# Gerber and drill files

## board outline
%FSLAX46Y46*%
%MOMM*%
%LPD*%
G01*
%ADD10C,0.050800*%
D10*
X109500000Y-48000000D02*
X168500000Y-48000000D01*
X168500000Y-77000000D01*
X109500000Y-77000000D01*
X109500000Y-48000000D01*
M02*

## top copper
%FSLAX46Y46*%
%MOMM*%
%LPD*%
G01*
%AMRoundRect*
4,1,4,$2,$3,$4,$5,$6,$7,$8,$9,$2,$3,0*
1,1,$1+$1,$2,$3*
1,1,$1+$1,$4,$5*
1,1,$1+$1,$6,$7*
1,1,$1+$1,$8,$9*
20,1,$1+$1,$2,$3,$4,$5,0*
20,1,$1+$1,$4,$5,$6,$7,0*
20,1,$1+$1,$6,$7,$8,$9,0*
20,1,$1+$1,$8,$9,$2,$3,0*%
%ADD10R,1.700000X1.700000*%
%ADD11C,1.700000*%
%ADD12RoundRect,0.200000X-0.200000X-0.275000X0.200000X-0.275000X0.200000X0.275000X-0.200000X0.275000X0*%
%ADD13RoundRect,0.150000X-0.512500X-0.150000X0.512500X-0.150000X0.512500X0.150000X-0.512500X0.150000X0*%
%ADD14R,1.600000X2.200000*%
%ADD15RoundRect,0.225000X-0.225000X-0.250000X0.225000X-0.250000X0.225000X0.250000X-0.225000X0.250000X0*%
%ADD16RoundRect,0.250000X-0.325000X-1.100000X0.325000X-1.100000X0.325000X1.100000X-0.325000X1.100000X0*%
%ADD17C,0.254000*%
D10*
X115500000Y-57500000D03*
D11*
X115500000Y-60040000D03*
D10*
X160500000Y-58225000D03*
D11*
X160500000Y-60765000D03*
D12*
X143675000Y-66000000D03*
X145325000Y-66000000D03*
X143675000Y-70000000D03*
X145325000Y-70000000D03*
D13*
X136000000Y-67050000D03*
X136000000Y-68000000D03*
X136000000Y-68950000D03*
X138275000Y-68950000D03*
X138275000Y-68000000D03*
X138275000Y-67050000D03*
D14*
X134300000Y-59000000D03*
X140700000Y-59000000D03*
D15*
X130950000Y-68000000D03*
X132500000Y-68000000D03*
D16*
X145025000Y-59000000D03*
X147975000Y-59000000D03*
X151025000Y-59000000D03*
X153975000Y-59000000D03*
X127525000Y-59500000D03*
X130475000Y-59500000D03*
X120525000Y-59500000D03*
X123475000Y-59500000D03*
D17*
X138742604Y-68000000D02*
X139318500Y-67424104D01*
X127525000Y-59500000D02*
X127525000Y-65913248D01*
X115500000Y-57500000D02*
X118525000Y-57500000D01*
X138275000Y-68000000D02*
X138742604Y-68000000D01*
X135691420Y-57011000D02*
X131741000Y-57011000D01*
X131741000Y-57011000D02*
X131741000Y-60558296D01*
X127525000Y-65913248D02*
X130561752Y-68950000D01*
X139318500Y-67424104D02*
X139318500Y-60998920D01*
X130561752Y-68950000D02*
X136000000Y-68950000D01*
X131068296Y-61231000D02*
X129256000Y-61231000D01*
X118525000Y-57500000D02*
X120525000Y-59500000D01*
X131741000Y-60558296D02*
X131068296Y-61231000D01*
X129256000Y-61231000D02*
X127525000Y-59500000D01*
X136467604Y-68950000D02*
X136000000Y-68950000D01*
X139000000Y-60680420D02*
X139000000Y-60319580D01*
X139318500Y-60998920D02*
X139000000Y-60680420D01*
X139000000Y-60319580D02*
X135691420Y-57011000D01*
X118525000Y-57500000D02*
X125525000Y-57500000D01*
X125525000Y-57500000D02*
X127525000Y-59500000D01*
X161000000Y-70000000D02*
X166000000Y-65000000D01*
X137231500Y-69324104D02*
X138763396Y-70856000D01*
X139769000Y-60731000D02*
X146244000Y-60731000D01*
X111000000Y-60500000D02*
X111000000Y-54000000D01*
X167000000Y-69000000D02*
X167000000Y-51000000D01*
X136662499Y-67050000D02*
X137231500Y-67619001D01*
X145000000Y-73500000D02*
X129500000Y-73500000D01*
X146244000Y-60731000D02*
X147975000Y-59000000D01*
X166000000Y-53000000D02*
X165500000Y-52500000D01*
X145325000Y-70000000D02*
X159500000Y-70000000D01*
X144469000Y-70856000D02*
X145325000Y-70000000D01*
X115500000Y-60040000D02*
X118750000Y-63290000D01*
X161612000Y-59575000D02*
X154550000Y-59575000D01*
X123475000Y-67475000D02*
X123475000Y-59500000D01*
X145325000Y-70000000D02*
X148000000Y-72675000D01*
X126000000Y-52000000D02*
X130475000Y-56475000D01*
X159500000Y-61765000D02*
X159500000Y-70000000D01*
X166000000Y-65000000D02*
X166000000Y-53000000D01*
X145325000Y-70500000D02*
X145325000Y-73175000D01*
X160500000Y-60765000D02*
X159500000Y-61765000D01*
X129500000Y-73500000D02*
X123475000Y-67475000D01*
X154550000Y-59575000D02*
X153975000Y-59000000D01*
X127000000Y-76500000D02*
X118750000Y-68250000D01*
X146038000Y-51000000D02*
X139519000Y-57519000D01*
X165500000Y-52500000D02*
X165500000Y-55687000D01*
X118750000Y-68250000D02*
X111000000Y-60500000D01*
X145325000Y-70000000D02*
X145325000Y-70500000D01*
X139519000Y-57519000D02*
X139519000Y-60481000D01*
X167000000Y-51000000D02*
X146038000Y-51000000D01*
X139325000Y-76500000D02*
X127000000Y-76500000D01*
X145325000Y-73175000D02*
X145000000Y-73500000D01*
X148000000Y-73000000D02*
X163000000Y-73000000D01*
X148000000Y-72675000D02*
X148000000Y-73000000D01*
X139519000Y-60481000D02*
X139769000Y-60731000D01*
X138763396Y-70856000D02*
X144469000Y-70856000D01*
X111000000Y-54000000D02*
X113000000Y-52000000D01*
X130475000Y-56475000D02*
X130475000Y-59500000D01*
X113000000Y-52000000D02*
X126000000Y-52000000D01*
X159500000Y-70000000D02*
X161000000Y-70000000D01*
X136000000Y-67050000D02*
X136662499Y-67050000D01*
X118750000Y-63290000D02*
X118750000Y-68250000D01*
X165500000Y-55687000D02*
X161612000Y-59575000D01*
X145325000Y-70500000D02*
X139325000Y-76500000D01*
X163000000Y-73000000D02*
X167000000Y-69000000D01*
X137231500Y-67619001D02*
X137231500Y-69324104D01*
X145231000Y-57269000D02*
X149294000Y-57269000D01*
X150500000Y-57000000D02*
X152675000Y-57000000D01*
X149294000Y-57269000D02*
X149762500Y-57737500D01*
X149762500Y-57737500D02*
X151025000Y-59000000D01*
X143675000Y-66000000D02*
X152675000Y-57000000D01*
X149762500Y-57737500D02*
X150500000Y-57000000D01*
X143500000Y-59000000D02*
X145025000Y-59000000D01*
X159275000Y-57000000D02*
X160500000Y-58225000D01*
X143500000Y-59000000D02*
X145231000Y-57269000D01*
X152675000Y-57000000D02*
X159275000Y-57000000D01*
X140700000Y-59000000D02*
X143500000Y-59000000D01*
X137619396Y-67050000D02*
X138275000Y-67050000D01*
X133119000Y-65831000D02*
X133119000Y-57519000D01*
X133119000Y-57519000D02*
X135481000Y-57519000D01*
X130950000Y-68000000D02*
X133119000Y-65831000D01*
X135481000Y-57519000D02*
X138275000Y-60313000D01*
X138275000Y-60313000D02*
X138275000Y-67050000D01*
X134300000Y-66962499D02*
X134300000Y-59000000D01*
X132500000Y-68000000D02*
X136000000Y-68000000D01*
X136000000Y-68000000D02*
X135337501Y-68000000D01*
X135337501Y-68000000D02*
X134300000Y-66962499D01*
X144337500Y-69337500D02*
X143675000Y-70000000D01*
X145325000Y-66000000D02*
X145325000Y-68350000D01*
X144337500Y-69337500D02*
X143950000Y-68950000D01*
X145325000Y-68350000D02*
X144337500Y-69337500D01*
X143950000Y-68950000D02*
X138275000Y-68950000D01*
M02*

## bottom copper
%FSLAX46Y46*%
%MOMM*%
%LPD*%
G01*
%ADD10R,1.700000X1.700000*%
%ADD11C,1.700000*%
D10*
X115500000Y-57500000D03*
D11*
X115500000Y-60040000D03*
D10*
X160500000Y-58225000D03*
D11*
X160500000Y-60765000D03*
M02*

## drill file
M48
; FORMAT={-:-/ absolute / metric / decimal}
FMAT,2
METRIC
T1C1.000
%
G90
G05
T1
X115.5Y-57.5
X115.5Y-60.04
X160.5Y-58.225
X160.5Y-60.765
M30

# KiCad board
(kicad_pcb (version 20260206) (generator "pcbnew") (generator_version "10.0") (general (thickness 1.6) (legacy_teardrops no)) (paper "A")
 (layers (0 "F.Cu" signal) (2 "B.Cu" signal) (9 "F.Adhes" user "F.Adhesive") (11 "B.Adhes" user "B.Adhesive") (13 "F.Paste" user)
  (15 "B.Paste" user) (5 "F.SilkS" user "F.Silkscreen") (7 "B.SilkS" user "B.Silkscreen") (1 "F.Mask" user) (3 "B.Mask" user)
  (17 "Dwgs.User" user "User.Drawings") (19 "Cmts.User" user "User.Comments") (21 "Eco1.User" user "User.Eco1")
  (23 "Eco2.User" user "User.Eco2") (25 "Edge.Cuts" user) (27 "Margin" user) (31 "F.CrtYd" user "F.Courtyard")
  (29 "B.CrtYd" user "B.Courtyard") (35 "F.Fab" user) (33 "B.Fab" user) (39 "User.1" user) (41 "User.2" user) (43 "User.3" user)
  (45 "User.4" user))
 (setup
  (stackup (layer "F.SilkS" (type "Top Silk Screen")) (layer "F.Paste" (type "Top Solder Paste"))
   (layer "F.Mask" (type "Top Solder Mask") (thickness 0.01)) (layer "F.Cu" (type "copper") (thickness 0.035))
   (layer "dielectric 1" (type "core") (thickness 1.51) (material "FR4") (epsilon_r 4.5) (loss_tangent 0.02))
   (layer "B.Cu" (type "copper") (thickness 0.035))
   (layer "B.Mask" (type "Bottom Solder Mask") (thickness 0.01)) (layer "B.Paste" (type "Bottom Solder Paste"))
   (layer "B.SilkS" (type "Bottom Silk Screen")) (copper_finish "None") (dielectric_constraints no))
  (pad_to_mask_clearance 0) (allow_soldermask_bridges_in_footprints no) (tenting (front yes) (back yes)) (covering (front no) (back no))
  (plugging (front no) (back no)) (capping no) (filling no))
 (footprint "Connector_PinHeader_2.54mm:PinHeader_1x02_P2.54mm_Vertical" (layer "F.Cu") (at 115.5 57.5)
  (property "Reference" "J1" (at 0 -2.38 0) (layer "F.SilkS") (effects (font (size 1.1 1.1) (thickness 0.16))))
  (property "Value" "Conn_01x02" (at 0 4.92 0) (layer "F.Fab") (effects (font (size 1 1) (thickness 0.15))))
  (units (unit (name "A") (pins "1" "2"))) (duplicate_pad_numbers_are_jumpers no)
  (pad "1" thru_hole rect (at 0 0) (size 1.7 1.7) (drill 1) (layers "*.Cu" "*.Mask") (remove_unused_layers no) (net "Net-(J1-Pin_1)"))
  (pad "2" thru_hole circle (at 0 2.54) (size 1.7 1.7) (drill 1) (layers "*.Cu" "*.Mask") (remove_unused_layers no) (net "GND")))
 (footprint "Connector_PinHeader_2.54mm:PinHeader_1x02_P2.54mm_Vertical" (layer "F.Cu") (at 160.5 58.225)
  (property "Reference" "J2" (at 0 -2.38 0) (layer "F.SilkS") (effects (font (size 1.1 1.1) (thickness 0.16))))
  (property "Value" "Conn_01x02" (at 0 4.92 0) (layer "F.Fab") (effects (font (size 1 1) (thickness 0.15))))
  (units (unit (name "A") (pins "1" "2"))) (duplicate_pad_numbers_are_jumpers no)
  (pad "1" thru_hole rect (at 0 0) (size 1.7 1.7) (drill 1) (layers "*.Cu" "*.Mask") (remove_unused_layers no) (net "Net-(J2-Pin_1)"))
  (pad "2" thru_hole circle (at 0 2.54) (size 1.7 1.7) (drill 1) (layers "*.Cu" "*.Mask") (remove_unused_layers no) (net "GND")))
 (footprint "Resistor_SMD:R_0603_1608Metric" (layer "F.Cu") (at 144.5 66)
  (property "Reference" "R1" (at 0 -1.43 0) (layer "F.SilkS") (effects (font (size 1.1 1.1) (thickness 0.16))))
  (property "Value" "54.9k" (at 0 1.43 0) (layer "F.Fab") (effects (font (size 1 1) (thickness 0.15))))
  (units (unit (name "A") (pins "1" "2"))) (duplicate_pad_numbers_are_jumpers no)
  (pad "1" smd roundrect (at -0.825 0) (size 0.8 0.95) (layers "F.Cu" "F.Mask" "F.Paste") (roundrect_rratio 0.25) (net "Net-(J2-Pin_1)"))
  (pad "2" smd roundrect (at 0.825 0) (size 0.8 0.95) (layers "F.Cu" "F.Mask" "F.Paste") (roundrect_rratio 0.25) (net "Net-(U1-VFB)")))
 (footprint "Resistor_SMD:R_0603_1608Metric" (layer "F.Cu") (at 144.5 70)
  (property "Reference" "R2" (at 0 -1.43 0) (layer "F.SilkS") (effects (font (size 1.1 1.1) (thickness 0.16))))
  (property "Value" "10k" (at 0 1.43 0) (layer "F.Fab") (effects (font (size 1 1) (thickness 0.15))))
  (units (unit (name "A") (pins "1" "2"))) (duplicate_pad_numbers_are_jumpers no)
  (pad "1" smd roundrect (at -0.825 0) (size 0.8 0.95) (layers "F.Cu" "F.Mask" "F.Paste") (roundrect_rratio 0.25) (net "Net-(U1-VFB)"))
  (pad "2" smd roundrect (at 0.825 0) (size 0.8 0.95) (layers "F.Cu" "F.Mask" "F.Paste") (roundrect_rratio 0.25) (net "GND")))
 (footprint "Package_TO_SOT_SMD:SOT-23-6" (layer "F.Cu") (at 137.1375 68)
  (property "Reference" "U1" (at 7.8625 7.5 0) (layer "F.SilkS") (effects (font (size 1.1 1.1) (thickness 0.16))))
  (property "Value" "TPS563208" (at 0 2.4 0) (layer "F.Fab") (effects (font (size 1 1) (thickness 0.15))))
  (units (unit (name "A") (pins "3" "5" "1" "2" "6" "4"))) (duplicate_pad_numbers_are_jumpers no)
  (pad "1" smd roundrect (at -1.1375 -0.95) (size 1.325 0.6) (layers "F.Cu" "F.Mask" "F.Paste") (roundrect_rratio 0.25) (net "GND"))
  (pad "2" smd roundrect (at -1.1375 0) (size 1.325 0.6) (layers "F.Cu" "F.Mask" "F.Paste") (roundrect_rratio 0.25) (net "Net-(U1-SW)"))
  (pad "3" smd roundrect (at -1.1375 0.95) (size 1.325 0.6) (layers "F.Cu" "F.Mask" "F.Paste") (roundrect_rratio 0.25)
   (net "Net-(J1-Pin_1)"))
  (pad "4" smd roundrect (at 1.1375 0.95) (size 1.325 0.6) (layers "F.Cu" "F.Mask" "F.Paste") (roundrect_rratio 0.25) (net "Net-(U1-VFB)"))
  (pad "5" smd roundrect (at 1.1375 0) (size 1.325 0.6) (layers "F.Cu" "F.Mask" "F.Paste") (roundrect_rratio 0.25) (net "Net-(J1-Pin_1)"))
  (pad "6" smd roundrect (at 1.1375 -0.95) (size 1.325 0.6) (layers "F.Cu" "F.Mask" "F.Paste") (roundrect_rratio 0.25) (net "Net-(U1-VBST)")))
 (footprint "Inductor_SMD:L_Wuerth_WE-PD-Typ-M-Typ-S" (layer "F.Cu") (at 137.5 59)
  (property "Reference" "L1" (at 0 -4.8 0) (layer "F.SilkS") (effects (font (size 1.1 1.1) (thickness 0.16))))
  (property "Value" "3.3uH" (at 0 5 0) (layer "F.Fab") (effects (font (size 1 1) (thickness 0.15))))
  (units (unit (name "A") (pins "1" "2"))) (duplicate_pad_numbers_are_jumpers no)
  (pad "1" smd rect (at -3.2 0) (size 1.6 2.2) (layers "F.Cu" "F.Mask" "F.Paste") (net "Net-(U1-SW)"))
  (pad "2" smd rect (at 3.2 0) (size 1.6 2.2) (layers "F.Cu" "F.Mask" "F.Paste") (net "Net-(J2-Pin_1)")))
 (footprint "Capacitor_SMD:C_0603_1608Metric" (layer "F.Cu") (at 131.725 68)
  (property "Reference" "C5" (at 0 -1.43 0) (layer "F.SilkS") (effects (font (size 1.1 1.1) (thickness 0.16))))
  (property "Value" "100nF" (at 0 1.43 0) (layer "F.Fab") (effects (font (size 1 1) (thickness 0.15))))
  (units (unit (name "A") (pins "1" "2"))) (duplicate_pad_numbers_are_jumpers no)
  (pad "1" smd roundrect (at -0.775 0) (size 0.9 0.95) (layers "F.Cu" "F.Mask" "F.Paste") (roundrect_rratio 0.25) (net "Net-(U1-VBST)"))
  (pad "2" smd roundrect (at 0.775 0) (size 0.9 0.95) (layers "F.Cu" "F.Mask" "F.Paste") (roundrect_rratio 0.25) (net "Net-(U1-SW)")))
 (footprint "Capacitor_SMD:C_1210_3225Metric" (layer "F.Cu") (at 146.5 59)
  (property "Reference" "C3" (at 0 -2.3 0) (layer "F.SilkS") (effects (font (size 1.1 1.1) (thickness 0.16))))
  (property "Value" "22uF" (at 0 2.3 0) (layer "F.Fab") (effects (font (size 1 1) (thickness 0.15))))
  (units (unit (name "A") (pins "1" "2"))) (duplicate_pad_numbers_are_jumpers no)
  (pad "1" smd roundrect (at -1.475 0) (size 1.15 2.7) (layers "F.Cu" "F.Mask" "F.Paste") (roundrect_rratio 0.217391) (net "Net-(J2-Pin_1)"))
  (pad "2" smd roundrect (at 1.475 0) (size 1.15 2.7) (layers "F.Cu" "F.Mask" "F.Paste") (roundrect_rratio 0.217391) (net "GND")))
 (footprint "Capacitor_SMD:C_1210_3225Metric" (layer "F.Cu") (at 152.5 59)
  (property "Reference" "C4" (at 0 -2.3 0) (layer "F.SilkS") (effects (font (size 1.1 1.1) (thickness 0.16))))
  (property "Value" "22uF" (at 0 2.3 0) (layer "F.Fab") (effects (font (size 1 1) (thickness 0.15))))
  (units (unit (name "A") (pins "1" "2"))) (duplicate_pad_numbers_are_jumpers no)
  (pad "1" smd roundrect (at -1.475 0) (size 1.15 2.7) (layers "F.Cu" "F.Mask" "F.Paste") (roundrect_rratio 0.217391) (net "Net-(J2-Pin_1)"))
  (pad "2" smd roundrect (at 1.475 0) (size 1.15 2.7) (layers "F.Cu" "F.Mask" "F.Paste") (roundrect_rratio 0.217391) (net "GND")))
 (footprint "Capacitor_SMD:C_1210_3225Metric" (layer "F.Cu") (at 129 59.5)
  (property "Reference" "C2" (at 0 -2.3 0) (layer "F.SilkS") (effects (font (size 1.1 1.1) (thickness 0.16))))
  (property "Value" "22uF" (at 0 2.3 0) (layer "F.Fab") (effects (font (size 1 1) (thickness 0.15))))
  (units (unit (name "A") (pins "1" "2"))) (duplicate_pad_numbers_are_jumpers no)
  (pad "1" smd roundrect (at -1.475 0) (size 1.15 2.7) (layers "F.Cu" "F.Mask" "F.Paste") (roundrect_rratio 0.217391) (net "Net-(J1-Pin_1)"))
  (pad "2" smd roundrect (at 1.475 0) (size 1.15 2.7) (layers "F.Cu" "F.Mask" "F.Paste") (roundrect_rratio 0.217391) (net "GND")))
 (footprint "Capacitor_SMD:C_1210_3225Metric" (layer "F.Cu") (at 122 59.5)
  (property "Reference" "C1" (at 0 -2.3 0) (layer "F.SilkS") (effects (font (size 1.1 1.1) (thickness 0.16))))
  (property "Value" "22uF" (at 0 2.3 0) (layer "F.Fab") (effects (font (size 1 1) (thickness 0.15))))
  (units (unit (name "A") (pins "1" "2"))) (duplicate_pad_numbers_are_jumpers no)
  (pad "1" smd roundrect (at -1.475 0) (size 1.15 2.7) (layers "F.Cu" "F.Mask" "F.Paste") (roundrect_rratio 0.217391) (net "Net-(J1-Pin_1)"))
  (pad "2" smd roundrect (at 1.475 0) (size 1.15 2.7) (layers "F.Cu" "F.Mask" "F.Paste") (roundrect_rratio 0.217391) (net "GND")))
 (gr_rect (start 109.5 48) (end 168.5 77) (stroke (width 0.0508) (type default)) (fill no) (layer "Edge.Cuts"))
 (segment (start 138.742604 68) (end 139.3185 67.424104) (width 0.254) (layer "F.Cu") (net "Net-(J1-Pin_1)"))
 (segment (start 127.525 59.5) (end 127.525 65.913248) (width 0.254) (layer "F.Cu") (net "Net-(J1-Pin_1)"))
 (segment (start 115.5 57.5) (end 118.525 57.5) (width 0.254) (layer "F.Cu") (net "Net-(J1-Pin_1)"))
 (segment (start 138.275 68) (end 138.742604 68) (width 0.254) (layer "F.Cu") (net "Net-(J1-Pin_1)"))
 (segment (start 135.69142 57.011) (end 131.741 57.011) (width 0.254) (layer "F.Cu") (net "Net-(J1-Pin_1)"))
 (segment (start 131.741 57.011) (end 131.741 60.558296) (width 0.254) (layer "F.Cu") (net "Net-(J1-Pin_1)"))
 (segment (start 127.525 65.913248) (end 130.561752 68.95) (width 0.254) (layer "F.Cu") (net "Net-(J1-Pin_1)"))
 (segment (start 139.3185 67.424104) (end 139.3185 60.99892) (width 0.254) (layer "F.Cu") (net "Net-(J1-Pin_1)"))
 (segment (start 130.561752 68.95) (end 136 68.95) (width 0.254) (layer "F.Cu") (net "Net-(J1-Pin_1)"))
 (segment (start 131.068296 61.231) (end 129.256 61.231) (width 0.254) (layer "F.Cu") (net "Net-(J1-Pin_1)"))
 (segment (start 118.525 57.5) (end 120.525 59.5) (width 0.254) (layer "F.Cu") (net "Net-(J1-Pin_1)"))
 (segment (start 131.741 60.558296) (end 131.068296 61.231) (width 0.254) (layer "F.Cu") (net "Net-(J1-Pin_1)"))
 (segment (start 129.256 61.231) (end 127.525 59.5) (width 0.254) (layer "F.Cu") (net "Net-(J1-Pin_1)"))
 (segment (start 136.467604 68.95) (end 136 68.95) (width 0.254) (layer "F.Cu") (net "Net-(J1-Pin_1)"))
 (segment (start 139 60.68042) (end 139 60.31958) (width 0.254) (layer "F.Cu") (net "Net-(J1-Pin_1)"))
 (segment (start 139.3185 60.99892) (end 139 60.68042) (width 0.254) (layer "F.Cu") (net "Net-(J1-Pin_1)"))
 (segment (start 139 60.31958) (end 135.69142 57.011) (width 0.254) (layer "F.Cu") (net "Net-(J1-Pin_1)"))
 (segment (start 118.525 57.5) (end 125.525 57.5) (width 0.254) (layer "F.Cu") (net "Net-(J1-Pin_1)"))
 (segment (start 125.525 57.5) (end 127.525 59.5) (width 0.254) (layer "F.Cu") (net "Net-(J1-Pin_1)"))
 (segment (start 161 70) (end 166 65) (width 0.254) (layer "F.Cu") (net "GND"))
 (segment (start 137.2315 69.324104) (end 138.763396 70.856) (width 0.254) (layer "F.Cu") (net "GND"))
 (segment (start 139.769 60.731) (end 146.244 60.731) (width 0.254) (layer "F.Cu") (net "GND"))
 (segment (start 111 60.5) (end 111 54) (width 0.254) (layer "F.Cu") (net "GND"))
 (segment (start 167 69) (end 167 51) (width 0.254) (layer "F.Cu") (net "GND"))
 (segment (start 136.662499 67.05) (end 137.2315 67.619001) (width 0.254) (layer "F.Cu") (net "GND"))
 (segment (start 145 73.5) (end 129.5 73.5) (width 0.254) (layer "F.Cu") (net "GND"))
 (segment (start 146.244 60.731) (end 147.975 59) (width 0.254) (layer "F.Cu") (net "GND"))
 (segment (start 166 53) (end 165.5 52.5) (width 0.254) (layer "F.Cu") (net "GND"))
 (segment (start 145.325 70) (end 159.5 70) (width 0.254) (layer "F.Cu") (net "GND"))
 (segment (start 144.469 70.856) (end 145.325 70) (width 0.254) (layer "F.Cu") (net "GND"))
 (segment (start 115.5 60.04) (end 118.75 63.29) (width 0.254) (layer "F.Cu") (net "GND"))
 (segment (start 161.612 59.575) (end 154.55 59.575) (width 0.254) (layer "F.Cu") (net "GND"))
 (segment (start 123.475 67.475) (end 123.475 59.5) (width 0.254) (layer "F.Cu") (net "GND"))
 (segment (start 145.325 70) (end 148 72.675) (width 0.254) (layer "F.Cu") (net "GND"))
 (segment (start 126 52) (end 130.475 56.475) (width 0.254) (layer "F.Cu") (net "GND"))
 (segment (start 159.5 61.765) (end 159.5 70) (width 0.254) (layer "F.Cu") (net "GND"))
 (segment (start 166 65) (end 166 53) (width 0.254) (layer "F.Cu") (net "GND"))
 (segment (start 145.325 70.5) (end 145.325 73.175) (width 0.254) (layer "F.Cu") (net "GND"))
 (segment (start 160.5 60.765) (end 159.5 61.765) (width 0.254) (layer "F.Cu") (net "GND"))
 (segment (start 129.5 73.5) (end 123.475 67.475) (width 0.254) (layer "F.Cu") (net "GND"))
 (segment (start 154.55 59.575) (end 153.975 59) (width 0.254) (layer "F.Cu") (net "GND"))
 (segment (start 127 76.5) (end 118.75 68.25) (width 0.254) (layer "F.Cu") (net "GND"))
 (segment (start 146.038 51) (end 139.519 57.519) (width 0.254) (layer "F.Cu") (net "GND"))
 (segment (start 165.5 52.5) (end 165.5 55.687) (width 0.254) (layer "F.Cu") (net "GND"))
 (segment (start 118.75 68.25) (end 111 60.5) (width 0.254) (layer "F.Cu") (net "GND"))
 (segment (start 145.325 70) (end 145.325 70.5) (width 0.254) (layer "F.Cu") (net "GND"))
 (segment (start 139.519 57.519) (end 139.519 60.481) (width 0.254) (layer "F.Cu") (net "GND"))
 (segment (start 167 51) (end 146.038 51) (width 0.254) (layer "F.Cu") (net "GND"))
 (segment (start 139.325 76.5) (end 127 76.5) (width 0.254) (layer "F.Cu") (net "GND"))
 (segment (start 145.325 73.175) (end 145 73.5) (width 0.254) (layer "F.Cu") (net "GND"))
 (segment (start 148 73) (end 163 73) (width 0.254) (layer "F.Cu") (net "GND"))
 (segment (start 148 72.675) (end 148 73) (width 0.254) (layer "F.Cu") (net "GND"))
 (segment (start 139.519 60.481) (end 139.769 60.731) (width 0.254) (layer "F.Cu") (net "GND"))
 (segment (start 138.763396 70.856) (end 144.469 70.856) (width 0.254) (layer "F.Cu") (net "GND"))
 (segment (start 111 54) (end 113 52) (width 0.254) (layer "F.Cu") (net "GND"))
 (segment (start 130.475 56.475) (end 130.475 59.5) (width 0.254) (layer "F.Cu") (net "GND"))
 (segment (start 113 52) (end 126 52) (width 0.254) (layer "F.Cu") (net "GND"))
 (segment (start 159.5 70) (end 161 70) (width 0.254) (layer "F.Cu") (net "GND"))
 (segment (start 136 67.05) (end 136.662499 67.05) (width 0.254) (layer "F.Cu") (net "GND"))
 (segment (start 118.75 63.29) (end 118.75 68.25) (width 0.254) (layer "F.Cu") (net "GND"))
 (segment (start 165.5 55.687) (end 161.612 59.575) (width 0.254) (layer "F.Cu") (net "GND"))
 (segment (start 145.325 70.5) (end 139.325 76.5) (width 0.254) (layer "F.Cu") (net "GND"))
 (segment (start 163 73) (end 167 69) (width 0.254) (layer "F.Cu") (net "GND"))
 (segment (start 137.2315 67.619001) (end 137.2315 69.324104) (width 0.254) (layer "F.Cu") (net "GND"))
 (segment (start 145.231 57.269) (end 149.294 57.269) (width 0.254) (layer "F.Cu") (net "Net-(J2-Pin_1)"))
 (segment (start 150.5 57) (end 152.675 57) (width 0.254) (layer "F.Cu") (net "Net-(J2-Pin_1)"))
 (segment (start 149.294 57.269) (end 149.7625 57.7375) (width 0.254) (layer "F.Cu") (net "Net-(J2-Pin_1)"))
 (segment (start 149.7625 57.7375) (end 151.025 59) (width 0.254) (layer "F.Cu") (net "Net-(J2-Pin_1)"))
 (segment (start 143.675 66) (end 152.675 57) (width 0.254) (layer "F.Cu") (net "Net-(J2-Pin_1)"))
 (segment (start 149.7625 57.7375) (end 150.5 57) (width 0.254) (layer "F.Cu") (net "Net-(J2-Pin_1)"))
 (segment (start 143.5 59) (end 145.025 59) (width 0.254) (layer "F.Cu") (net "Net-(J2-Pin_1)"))
 (segment (start 159.275 57) (end 160.5 58.225) (width 0.254) (layer "F.Cu") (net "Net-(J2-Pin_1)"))
 (segment (start 143.5 59) (end 145.231 57.269) (width 0.254) (layer "F.Cu") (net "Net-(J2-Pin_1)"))
 (segment (start 152.675 57) (end 159.275 57) (width 0.254) (layer "F.Cu") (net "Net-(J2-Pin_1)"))
 (segment (start 140.7 59) (end 143.5 59) (width 0.254) (layer "F.Cu") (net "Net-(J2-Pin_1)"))
 (segment (start 137.619396 67.05) (end 138.275 67.05) (width 0.254) (layer "F.Cu") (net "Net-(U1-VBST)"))
 (segment (start 133.119 65.831) (end 133.119 57.519) (width 0.254) (layer "F.Cu") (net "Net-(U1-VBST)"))
 (segment (start 133.119 57.519) (end 135.481 57.519) (width 0.254) (layer "F.Cu") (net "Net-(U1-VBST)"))
 (segment (start 130.95 68) (end 133.119 65.831) (width 0.254) (layer "F.Cu") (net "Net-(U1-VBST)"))
 (segment (start 135.481 57.519) (end 138.275 60.313) (width 0.254) (layer "F.Cu") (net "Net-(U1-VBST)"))
 (segment (start 138.275 60.313) (end 138.275 67.05) (width 0.254) (layer "F.Cu") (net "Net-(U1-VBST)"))
 (segment (start 134.3 66.962499) (end 134.3 59) (width 0.254) (layer "F.Cu") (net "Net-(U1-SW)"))
 (segment (start 132.5 68) (end 136 68) (width 0.254) (layer "F.Cu") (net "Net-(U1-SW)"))
 (segment (start 136 68) (end 135.337501 68) (width 0.254) (layer "F.Cu") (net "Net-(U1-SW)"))
 (segment (start 135.337501 68) (end 134.3 66.962499) (width 0.254) (layer "F.Cu") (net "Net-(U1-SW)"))
 (segment (start 144.3375 69.3375) (end 143.675 70) (width 0.254) (layer "F.Cu") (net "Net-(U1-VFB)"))
 (segment (start 145.325 66) (end 145.325 68.35) (width 0.254) (layer "F.Cu") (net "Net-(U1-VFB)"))
 (segment (start 144.3375 69.3375) (end 143.95 68.95) (width 0.254) (layer "F.Cu") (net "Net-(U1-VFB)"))
 (segment (start 145.325 68.35) (end 144.3375 69.3375) (width 0.254) (layer "F.Cu") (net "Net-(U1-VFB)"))
 (segment (start 143.95 68.95) (end 138.275 68.95) (width 0.254) (layer "F.Cu") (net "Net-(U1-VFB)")))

